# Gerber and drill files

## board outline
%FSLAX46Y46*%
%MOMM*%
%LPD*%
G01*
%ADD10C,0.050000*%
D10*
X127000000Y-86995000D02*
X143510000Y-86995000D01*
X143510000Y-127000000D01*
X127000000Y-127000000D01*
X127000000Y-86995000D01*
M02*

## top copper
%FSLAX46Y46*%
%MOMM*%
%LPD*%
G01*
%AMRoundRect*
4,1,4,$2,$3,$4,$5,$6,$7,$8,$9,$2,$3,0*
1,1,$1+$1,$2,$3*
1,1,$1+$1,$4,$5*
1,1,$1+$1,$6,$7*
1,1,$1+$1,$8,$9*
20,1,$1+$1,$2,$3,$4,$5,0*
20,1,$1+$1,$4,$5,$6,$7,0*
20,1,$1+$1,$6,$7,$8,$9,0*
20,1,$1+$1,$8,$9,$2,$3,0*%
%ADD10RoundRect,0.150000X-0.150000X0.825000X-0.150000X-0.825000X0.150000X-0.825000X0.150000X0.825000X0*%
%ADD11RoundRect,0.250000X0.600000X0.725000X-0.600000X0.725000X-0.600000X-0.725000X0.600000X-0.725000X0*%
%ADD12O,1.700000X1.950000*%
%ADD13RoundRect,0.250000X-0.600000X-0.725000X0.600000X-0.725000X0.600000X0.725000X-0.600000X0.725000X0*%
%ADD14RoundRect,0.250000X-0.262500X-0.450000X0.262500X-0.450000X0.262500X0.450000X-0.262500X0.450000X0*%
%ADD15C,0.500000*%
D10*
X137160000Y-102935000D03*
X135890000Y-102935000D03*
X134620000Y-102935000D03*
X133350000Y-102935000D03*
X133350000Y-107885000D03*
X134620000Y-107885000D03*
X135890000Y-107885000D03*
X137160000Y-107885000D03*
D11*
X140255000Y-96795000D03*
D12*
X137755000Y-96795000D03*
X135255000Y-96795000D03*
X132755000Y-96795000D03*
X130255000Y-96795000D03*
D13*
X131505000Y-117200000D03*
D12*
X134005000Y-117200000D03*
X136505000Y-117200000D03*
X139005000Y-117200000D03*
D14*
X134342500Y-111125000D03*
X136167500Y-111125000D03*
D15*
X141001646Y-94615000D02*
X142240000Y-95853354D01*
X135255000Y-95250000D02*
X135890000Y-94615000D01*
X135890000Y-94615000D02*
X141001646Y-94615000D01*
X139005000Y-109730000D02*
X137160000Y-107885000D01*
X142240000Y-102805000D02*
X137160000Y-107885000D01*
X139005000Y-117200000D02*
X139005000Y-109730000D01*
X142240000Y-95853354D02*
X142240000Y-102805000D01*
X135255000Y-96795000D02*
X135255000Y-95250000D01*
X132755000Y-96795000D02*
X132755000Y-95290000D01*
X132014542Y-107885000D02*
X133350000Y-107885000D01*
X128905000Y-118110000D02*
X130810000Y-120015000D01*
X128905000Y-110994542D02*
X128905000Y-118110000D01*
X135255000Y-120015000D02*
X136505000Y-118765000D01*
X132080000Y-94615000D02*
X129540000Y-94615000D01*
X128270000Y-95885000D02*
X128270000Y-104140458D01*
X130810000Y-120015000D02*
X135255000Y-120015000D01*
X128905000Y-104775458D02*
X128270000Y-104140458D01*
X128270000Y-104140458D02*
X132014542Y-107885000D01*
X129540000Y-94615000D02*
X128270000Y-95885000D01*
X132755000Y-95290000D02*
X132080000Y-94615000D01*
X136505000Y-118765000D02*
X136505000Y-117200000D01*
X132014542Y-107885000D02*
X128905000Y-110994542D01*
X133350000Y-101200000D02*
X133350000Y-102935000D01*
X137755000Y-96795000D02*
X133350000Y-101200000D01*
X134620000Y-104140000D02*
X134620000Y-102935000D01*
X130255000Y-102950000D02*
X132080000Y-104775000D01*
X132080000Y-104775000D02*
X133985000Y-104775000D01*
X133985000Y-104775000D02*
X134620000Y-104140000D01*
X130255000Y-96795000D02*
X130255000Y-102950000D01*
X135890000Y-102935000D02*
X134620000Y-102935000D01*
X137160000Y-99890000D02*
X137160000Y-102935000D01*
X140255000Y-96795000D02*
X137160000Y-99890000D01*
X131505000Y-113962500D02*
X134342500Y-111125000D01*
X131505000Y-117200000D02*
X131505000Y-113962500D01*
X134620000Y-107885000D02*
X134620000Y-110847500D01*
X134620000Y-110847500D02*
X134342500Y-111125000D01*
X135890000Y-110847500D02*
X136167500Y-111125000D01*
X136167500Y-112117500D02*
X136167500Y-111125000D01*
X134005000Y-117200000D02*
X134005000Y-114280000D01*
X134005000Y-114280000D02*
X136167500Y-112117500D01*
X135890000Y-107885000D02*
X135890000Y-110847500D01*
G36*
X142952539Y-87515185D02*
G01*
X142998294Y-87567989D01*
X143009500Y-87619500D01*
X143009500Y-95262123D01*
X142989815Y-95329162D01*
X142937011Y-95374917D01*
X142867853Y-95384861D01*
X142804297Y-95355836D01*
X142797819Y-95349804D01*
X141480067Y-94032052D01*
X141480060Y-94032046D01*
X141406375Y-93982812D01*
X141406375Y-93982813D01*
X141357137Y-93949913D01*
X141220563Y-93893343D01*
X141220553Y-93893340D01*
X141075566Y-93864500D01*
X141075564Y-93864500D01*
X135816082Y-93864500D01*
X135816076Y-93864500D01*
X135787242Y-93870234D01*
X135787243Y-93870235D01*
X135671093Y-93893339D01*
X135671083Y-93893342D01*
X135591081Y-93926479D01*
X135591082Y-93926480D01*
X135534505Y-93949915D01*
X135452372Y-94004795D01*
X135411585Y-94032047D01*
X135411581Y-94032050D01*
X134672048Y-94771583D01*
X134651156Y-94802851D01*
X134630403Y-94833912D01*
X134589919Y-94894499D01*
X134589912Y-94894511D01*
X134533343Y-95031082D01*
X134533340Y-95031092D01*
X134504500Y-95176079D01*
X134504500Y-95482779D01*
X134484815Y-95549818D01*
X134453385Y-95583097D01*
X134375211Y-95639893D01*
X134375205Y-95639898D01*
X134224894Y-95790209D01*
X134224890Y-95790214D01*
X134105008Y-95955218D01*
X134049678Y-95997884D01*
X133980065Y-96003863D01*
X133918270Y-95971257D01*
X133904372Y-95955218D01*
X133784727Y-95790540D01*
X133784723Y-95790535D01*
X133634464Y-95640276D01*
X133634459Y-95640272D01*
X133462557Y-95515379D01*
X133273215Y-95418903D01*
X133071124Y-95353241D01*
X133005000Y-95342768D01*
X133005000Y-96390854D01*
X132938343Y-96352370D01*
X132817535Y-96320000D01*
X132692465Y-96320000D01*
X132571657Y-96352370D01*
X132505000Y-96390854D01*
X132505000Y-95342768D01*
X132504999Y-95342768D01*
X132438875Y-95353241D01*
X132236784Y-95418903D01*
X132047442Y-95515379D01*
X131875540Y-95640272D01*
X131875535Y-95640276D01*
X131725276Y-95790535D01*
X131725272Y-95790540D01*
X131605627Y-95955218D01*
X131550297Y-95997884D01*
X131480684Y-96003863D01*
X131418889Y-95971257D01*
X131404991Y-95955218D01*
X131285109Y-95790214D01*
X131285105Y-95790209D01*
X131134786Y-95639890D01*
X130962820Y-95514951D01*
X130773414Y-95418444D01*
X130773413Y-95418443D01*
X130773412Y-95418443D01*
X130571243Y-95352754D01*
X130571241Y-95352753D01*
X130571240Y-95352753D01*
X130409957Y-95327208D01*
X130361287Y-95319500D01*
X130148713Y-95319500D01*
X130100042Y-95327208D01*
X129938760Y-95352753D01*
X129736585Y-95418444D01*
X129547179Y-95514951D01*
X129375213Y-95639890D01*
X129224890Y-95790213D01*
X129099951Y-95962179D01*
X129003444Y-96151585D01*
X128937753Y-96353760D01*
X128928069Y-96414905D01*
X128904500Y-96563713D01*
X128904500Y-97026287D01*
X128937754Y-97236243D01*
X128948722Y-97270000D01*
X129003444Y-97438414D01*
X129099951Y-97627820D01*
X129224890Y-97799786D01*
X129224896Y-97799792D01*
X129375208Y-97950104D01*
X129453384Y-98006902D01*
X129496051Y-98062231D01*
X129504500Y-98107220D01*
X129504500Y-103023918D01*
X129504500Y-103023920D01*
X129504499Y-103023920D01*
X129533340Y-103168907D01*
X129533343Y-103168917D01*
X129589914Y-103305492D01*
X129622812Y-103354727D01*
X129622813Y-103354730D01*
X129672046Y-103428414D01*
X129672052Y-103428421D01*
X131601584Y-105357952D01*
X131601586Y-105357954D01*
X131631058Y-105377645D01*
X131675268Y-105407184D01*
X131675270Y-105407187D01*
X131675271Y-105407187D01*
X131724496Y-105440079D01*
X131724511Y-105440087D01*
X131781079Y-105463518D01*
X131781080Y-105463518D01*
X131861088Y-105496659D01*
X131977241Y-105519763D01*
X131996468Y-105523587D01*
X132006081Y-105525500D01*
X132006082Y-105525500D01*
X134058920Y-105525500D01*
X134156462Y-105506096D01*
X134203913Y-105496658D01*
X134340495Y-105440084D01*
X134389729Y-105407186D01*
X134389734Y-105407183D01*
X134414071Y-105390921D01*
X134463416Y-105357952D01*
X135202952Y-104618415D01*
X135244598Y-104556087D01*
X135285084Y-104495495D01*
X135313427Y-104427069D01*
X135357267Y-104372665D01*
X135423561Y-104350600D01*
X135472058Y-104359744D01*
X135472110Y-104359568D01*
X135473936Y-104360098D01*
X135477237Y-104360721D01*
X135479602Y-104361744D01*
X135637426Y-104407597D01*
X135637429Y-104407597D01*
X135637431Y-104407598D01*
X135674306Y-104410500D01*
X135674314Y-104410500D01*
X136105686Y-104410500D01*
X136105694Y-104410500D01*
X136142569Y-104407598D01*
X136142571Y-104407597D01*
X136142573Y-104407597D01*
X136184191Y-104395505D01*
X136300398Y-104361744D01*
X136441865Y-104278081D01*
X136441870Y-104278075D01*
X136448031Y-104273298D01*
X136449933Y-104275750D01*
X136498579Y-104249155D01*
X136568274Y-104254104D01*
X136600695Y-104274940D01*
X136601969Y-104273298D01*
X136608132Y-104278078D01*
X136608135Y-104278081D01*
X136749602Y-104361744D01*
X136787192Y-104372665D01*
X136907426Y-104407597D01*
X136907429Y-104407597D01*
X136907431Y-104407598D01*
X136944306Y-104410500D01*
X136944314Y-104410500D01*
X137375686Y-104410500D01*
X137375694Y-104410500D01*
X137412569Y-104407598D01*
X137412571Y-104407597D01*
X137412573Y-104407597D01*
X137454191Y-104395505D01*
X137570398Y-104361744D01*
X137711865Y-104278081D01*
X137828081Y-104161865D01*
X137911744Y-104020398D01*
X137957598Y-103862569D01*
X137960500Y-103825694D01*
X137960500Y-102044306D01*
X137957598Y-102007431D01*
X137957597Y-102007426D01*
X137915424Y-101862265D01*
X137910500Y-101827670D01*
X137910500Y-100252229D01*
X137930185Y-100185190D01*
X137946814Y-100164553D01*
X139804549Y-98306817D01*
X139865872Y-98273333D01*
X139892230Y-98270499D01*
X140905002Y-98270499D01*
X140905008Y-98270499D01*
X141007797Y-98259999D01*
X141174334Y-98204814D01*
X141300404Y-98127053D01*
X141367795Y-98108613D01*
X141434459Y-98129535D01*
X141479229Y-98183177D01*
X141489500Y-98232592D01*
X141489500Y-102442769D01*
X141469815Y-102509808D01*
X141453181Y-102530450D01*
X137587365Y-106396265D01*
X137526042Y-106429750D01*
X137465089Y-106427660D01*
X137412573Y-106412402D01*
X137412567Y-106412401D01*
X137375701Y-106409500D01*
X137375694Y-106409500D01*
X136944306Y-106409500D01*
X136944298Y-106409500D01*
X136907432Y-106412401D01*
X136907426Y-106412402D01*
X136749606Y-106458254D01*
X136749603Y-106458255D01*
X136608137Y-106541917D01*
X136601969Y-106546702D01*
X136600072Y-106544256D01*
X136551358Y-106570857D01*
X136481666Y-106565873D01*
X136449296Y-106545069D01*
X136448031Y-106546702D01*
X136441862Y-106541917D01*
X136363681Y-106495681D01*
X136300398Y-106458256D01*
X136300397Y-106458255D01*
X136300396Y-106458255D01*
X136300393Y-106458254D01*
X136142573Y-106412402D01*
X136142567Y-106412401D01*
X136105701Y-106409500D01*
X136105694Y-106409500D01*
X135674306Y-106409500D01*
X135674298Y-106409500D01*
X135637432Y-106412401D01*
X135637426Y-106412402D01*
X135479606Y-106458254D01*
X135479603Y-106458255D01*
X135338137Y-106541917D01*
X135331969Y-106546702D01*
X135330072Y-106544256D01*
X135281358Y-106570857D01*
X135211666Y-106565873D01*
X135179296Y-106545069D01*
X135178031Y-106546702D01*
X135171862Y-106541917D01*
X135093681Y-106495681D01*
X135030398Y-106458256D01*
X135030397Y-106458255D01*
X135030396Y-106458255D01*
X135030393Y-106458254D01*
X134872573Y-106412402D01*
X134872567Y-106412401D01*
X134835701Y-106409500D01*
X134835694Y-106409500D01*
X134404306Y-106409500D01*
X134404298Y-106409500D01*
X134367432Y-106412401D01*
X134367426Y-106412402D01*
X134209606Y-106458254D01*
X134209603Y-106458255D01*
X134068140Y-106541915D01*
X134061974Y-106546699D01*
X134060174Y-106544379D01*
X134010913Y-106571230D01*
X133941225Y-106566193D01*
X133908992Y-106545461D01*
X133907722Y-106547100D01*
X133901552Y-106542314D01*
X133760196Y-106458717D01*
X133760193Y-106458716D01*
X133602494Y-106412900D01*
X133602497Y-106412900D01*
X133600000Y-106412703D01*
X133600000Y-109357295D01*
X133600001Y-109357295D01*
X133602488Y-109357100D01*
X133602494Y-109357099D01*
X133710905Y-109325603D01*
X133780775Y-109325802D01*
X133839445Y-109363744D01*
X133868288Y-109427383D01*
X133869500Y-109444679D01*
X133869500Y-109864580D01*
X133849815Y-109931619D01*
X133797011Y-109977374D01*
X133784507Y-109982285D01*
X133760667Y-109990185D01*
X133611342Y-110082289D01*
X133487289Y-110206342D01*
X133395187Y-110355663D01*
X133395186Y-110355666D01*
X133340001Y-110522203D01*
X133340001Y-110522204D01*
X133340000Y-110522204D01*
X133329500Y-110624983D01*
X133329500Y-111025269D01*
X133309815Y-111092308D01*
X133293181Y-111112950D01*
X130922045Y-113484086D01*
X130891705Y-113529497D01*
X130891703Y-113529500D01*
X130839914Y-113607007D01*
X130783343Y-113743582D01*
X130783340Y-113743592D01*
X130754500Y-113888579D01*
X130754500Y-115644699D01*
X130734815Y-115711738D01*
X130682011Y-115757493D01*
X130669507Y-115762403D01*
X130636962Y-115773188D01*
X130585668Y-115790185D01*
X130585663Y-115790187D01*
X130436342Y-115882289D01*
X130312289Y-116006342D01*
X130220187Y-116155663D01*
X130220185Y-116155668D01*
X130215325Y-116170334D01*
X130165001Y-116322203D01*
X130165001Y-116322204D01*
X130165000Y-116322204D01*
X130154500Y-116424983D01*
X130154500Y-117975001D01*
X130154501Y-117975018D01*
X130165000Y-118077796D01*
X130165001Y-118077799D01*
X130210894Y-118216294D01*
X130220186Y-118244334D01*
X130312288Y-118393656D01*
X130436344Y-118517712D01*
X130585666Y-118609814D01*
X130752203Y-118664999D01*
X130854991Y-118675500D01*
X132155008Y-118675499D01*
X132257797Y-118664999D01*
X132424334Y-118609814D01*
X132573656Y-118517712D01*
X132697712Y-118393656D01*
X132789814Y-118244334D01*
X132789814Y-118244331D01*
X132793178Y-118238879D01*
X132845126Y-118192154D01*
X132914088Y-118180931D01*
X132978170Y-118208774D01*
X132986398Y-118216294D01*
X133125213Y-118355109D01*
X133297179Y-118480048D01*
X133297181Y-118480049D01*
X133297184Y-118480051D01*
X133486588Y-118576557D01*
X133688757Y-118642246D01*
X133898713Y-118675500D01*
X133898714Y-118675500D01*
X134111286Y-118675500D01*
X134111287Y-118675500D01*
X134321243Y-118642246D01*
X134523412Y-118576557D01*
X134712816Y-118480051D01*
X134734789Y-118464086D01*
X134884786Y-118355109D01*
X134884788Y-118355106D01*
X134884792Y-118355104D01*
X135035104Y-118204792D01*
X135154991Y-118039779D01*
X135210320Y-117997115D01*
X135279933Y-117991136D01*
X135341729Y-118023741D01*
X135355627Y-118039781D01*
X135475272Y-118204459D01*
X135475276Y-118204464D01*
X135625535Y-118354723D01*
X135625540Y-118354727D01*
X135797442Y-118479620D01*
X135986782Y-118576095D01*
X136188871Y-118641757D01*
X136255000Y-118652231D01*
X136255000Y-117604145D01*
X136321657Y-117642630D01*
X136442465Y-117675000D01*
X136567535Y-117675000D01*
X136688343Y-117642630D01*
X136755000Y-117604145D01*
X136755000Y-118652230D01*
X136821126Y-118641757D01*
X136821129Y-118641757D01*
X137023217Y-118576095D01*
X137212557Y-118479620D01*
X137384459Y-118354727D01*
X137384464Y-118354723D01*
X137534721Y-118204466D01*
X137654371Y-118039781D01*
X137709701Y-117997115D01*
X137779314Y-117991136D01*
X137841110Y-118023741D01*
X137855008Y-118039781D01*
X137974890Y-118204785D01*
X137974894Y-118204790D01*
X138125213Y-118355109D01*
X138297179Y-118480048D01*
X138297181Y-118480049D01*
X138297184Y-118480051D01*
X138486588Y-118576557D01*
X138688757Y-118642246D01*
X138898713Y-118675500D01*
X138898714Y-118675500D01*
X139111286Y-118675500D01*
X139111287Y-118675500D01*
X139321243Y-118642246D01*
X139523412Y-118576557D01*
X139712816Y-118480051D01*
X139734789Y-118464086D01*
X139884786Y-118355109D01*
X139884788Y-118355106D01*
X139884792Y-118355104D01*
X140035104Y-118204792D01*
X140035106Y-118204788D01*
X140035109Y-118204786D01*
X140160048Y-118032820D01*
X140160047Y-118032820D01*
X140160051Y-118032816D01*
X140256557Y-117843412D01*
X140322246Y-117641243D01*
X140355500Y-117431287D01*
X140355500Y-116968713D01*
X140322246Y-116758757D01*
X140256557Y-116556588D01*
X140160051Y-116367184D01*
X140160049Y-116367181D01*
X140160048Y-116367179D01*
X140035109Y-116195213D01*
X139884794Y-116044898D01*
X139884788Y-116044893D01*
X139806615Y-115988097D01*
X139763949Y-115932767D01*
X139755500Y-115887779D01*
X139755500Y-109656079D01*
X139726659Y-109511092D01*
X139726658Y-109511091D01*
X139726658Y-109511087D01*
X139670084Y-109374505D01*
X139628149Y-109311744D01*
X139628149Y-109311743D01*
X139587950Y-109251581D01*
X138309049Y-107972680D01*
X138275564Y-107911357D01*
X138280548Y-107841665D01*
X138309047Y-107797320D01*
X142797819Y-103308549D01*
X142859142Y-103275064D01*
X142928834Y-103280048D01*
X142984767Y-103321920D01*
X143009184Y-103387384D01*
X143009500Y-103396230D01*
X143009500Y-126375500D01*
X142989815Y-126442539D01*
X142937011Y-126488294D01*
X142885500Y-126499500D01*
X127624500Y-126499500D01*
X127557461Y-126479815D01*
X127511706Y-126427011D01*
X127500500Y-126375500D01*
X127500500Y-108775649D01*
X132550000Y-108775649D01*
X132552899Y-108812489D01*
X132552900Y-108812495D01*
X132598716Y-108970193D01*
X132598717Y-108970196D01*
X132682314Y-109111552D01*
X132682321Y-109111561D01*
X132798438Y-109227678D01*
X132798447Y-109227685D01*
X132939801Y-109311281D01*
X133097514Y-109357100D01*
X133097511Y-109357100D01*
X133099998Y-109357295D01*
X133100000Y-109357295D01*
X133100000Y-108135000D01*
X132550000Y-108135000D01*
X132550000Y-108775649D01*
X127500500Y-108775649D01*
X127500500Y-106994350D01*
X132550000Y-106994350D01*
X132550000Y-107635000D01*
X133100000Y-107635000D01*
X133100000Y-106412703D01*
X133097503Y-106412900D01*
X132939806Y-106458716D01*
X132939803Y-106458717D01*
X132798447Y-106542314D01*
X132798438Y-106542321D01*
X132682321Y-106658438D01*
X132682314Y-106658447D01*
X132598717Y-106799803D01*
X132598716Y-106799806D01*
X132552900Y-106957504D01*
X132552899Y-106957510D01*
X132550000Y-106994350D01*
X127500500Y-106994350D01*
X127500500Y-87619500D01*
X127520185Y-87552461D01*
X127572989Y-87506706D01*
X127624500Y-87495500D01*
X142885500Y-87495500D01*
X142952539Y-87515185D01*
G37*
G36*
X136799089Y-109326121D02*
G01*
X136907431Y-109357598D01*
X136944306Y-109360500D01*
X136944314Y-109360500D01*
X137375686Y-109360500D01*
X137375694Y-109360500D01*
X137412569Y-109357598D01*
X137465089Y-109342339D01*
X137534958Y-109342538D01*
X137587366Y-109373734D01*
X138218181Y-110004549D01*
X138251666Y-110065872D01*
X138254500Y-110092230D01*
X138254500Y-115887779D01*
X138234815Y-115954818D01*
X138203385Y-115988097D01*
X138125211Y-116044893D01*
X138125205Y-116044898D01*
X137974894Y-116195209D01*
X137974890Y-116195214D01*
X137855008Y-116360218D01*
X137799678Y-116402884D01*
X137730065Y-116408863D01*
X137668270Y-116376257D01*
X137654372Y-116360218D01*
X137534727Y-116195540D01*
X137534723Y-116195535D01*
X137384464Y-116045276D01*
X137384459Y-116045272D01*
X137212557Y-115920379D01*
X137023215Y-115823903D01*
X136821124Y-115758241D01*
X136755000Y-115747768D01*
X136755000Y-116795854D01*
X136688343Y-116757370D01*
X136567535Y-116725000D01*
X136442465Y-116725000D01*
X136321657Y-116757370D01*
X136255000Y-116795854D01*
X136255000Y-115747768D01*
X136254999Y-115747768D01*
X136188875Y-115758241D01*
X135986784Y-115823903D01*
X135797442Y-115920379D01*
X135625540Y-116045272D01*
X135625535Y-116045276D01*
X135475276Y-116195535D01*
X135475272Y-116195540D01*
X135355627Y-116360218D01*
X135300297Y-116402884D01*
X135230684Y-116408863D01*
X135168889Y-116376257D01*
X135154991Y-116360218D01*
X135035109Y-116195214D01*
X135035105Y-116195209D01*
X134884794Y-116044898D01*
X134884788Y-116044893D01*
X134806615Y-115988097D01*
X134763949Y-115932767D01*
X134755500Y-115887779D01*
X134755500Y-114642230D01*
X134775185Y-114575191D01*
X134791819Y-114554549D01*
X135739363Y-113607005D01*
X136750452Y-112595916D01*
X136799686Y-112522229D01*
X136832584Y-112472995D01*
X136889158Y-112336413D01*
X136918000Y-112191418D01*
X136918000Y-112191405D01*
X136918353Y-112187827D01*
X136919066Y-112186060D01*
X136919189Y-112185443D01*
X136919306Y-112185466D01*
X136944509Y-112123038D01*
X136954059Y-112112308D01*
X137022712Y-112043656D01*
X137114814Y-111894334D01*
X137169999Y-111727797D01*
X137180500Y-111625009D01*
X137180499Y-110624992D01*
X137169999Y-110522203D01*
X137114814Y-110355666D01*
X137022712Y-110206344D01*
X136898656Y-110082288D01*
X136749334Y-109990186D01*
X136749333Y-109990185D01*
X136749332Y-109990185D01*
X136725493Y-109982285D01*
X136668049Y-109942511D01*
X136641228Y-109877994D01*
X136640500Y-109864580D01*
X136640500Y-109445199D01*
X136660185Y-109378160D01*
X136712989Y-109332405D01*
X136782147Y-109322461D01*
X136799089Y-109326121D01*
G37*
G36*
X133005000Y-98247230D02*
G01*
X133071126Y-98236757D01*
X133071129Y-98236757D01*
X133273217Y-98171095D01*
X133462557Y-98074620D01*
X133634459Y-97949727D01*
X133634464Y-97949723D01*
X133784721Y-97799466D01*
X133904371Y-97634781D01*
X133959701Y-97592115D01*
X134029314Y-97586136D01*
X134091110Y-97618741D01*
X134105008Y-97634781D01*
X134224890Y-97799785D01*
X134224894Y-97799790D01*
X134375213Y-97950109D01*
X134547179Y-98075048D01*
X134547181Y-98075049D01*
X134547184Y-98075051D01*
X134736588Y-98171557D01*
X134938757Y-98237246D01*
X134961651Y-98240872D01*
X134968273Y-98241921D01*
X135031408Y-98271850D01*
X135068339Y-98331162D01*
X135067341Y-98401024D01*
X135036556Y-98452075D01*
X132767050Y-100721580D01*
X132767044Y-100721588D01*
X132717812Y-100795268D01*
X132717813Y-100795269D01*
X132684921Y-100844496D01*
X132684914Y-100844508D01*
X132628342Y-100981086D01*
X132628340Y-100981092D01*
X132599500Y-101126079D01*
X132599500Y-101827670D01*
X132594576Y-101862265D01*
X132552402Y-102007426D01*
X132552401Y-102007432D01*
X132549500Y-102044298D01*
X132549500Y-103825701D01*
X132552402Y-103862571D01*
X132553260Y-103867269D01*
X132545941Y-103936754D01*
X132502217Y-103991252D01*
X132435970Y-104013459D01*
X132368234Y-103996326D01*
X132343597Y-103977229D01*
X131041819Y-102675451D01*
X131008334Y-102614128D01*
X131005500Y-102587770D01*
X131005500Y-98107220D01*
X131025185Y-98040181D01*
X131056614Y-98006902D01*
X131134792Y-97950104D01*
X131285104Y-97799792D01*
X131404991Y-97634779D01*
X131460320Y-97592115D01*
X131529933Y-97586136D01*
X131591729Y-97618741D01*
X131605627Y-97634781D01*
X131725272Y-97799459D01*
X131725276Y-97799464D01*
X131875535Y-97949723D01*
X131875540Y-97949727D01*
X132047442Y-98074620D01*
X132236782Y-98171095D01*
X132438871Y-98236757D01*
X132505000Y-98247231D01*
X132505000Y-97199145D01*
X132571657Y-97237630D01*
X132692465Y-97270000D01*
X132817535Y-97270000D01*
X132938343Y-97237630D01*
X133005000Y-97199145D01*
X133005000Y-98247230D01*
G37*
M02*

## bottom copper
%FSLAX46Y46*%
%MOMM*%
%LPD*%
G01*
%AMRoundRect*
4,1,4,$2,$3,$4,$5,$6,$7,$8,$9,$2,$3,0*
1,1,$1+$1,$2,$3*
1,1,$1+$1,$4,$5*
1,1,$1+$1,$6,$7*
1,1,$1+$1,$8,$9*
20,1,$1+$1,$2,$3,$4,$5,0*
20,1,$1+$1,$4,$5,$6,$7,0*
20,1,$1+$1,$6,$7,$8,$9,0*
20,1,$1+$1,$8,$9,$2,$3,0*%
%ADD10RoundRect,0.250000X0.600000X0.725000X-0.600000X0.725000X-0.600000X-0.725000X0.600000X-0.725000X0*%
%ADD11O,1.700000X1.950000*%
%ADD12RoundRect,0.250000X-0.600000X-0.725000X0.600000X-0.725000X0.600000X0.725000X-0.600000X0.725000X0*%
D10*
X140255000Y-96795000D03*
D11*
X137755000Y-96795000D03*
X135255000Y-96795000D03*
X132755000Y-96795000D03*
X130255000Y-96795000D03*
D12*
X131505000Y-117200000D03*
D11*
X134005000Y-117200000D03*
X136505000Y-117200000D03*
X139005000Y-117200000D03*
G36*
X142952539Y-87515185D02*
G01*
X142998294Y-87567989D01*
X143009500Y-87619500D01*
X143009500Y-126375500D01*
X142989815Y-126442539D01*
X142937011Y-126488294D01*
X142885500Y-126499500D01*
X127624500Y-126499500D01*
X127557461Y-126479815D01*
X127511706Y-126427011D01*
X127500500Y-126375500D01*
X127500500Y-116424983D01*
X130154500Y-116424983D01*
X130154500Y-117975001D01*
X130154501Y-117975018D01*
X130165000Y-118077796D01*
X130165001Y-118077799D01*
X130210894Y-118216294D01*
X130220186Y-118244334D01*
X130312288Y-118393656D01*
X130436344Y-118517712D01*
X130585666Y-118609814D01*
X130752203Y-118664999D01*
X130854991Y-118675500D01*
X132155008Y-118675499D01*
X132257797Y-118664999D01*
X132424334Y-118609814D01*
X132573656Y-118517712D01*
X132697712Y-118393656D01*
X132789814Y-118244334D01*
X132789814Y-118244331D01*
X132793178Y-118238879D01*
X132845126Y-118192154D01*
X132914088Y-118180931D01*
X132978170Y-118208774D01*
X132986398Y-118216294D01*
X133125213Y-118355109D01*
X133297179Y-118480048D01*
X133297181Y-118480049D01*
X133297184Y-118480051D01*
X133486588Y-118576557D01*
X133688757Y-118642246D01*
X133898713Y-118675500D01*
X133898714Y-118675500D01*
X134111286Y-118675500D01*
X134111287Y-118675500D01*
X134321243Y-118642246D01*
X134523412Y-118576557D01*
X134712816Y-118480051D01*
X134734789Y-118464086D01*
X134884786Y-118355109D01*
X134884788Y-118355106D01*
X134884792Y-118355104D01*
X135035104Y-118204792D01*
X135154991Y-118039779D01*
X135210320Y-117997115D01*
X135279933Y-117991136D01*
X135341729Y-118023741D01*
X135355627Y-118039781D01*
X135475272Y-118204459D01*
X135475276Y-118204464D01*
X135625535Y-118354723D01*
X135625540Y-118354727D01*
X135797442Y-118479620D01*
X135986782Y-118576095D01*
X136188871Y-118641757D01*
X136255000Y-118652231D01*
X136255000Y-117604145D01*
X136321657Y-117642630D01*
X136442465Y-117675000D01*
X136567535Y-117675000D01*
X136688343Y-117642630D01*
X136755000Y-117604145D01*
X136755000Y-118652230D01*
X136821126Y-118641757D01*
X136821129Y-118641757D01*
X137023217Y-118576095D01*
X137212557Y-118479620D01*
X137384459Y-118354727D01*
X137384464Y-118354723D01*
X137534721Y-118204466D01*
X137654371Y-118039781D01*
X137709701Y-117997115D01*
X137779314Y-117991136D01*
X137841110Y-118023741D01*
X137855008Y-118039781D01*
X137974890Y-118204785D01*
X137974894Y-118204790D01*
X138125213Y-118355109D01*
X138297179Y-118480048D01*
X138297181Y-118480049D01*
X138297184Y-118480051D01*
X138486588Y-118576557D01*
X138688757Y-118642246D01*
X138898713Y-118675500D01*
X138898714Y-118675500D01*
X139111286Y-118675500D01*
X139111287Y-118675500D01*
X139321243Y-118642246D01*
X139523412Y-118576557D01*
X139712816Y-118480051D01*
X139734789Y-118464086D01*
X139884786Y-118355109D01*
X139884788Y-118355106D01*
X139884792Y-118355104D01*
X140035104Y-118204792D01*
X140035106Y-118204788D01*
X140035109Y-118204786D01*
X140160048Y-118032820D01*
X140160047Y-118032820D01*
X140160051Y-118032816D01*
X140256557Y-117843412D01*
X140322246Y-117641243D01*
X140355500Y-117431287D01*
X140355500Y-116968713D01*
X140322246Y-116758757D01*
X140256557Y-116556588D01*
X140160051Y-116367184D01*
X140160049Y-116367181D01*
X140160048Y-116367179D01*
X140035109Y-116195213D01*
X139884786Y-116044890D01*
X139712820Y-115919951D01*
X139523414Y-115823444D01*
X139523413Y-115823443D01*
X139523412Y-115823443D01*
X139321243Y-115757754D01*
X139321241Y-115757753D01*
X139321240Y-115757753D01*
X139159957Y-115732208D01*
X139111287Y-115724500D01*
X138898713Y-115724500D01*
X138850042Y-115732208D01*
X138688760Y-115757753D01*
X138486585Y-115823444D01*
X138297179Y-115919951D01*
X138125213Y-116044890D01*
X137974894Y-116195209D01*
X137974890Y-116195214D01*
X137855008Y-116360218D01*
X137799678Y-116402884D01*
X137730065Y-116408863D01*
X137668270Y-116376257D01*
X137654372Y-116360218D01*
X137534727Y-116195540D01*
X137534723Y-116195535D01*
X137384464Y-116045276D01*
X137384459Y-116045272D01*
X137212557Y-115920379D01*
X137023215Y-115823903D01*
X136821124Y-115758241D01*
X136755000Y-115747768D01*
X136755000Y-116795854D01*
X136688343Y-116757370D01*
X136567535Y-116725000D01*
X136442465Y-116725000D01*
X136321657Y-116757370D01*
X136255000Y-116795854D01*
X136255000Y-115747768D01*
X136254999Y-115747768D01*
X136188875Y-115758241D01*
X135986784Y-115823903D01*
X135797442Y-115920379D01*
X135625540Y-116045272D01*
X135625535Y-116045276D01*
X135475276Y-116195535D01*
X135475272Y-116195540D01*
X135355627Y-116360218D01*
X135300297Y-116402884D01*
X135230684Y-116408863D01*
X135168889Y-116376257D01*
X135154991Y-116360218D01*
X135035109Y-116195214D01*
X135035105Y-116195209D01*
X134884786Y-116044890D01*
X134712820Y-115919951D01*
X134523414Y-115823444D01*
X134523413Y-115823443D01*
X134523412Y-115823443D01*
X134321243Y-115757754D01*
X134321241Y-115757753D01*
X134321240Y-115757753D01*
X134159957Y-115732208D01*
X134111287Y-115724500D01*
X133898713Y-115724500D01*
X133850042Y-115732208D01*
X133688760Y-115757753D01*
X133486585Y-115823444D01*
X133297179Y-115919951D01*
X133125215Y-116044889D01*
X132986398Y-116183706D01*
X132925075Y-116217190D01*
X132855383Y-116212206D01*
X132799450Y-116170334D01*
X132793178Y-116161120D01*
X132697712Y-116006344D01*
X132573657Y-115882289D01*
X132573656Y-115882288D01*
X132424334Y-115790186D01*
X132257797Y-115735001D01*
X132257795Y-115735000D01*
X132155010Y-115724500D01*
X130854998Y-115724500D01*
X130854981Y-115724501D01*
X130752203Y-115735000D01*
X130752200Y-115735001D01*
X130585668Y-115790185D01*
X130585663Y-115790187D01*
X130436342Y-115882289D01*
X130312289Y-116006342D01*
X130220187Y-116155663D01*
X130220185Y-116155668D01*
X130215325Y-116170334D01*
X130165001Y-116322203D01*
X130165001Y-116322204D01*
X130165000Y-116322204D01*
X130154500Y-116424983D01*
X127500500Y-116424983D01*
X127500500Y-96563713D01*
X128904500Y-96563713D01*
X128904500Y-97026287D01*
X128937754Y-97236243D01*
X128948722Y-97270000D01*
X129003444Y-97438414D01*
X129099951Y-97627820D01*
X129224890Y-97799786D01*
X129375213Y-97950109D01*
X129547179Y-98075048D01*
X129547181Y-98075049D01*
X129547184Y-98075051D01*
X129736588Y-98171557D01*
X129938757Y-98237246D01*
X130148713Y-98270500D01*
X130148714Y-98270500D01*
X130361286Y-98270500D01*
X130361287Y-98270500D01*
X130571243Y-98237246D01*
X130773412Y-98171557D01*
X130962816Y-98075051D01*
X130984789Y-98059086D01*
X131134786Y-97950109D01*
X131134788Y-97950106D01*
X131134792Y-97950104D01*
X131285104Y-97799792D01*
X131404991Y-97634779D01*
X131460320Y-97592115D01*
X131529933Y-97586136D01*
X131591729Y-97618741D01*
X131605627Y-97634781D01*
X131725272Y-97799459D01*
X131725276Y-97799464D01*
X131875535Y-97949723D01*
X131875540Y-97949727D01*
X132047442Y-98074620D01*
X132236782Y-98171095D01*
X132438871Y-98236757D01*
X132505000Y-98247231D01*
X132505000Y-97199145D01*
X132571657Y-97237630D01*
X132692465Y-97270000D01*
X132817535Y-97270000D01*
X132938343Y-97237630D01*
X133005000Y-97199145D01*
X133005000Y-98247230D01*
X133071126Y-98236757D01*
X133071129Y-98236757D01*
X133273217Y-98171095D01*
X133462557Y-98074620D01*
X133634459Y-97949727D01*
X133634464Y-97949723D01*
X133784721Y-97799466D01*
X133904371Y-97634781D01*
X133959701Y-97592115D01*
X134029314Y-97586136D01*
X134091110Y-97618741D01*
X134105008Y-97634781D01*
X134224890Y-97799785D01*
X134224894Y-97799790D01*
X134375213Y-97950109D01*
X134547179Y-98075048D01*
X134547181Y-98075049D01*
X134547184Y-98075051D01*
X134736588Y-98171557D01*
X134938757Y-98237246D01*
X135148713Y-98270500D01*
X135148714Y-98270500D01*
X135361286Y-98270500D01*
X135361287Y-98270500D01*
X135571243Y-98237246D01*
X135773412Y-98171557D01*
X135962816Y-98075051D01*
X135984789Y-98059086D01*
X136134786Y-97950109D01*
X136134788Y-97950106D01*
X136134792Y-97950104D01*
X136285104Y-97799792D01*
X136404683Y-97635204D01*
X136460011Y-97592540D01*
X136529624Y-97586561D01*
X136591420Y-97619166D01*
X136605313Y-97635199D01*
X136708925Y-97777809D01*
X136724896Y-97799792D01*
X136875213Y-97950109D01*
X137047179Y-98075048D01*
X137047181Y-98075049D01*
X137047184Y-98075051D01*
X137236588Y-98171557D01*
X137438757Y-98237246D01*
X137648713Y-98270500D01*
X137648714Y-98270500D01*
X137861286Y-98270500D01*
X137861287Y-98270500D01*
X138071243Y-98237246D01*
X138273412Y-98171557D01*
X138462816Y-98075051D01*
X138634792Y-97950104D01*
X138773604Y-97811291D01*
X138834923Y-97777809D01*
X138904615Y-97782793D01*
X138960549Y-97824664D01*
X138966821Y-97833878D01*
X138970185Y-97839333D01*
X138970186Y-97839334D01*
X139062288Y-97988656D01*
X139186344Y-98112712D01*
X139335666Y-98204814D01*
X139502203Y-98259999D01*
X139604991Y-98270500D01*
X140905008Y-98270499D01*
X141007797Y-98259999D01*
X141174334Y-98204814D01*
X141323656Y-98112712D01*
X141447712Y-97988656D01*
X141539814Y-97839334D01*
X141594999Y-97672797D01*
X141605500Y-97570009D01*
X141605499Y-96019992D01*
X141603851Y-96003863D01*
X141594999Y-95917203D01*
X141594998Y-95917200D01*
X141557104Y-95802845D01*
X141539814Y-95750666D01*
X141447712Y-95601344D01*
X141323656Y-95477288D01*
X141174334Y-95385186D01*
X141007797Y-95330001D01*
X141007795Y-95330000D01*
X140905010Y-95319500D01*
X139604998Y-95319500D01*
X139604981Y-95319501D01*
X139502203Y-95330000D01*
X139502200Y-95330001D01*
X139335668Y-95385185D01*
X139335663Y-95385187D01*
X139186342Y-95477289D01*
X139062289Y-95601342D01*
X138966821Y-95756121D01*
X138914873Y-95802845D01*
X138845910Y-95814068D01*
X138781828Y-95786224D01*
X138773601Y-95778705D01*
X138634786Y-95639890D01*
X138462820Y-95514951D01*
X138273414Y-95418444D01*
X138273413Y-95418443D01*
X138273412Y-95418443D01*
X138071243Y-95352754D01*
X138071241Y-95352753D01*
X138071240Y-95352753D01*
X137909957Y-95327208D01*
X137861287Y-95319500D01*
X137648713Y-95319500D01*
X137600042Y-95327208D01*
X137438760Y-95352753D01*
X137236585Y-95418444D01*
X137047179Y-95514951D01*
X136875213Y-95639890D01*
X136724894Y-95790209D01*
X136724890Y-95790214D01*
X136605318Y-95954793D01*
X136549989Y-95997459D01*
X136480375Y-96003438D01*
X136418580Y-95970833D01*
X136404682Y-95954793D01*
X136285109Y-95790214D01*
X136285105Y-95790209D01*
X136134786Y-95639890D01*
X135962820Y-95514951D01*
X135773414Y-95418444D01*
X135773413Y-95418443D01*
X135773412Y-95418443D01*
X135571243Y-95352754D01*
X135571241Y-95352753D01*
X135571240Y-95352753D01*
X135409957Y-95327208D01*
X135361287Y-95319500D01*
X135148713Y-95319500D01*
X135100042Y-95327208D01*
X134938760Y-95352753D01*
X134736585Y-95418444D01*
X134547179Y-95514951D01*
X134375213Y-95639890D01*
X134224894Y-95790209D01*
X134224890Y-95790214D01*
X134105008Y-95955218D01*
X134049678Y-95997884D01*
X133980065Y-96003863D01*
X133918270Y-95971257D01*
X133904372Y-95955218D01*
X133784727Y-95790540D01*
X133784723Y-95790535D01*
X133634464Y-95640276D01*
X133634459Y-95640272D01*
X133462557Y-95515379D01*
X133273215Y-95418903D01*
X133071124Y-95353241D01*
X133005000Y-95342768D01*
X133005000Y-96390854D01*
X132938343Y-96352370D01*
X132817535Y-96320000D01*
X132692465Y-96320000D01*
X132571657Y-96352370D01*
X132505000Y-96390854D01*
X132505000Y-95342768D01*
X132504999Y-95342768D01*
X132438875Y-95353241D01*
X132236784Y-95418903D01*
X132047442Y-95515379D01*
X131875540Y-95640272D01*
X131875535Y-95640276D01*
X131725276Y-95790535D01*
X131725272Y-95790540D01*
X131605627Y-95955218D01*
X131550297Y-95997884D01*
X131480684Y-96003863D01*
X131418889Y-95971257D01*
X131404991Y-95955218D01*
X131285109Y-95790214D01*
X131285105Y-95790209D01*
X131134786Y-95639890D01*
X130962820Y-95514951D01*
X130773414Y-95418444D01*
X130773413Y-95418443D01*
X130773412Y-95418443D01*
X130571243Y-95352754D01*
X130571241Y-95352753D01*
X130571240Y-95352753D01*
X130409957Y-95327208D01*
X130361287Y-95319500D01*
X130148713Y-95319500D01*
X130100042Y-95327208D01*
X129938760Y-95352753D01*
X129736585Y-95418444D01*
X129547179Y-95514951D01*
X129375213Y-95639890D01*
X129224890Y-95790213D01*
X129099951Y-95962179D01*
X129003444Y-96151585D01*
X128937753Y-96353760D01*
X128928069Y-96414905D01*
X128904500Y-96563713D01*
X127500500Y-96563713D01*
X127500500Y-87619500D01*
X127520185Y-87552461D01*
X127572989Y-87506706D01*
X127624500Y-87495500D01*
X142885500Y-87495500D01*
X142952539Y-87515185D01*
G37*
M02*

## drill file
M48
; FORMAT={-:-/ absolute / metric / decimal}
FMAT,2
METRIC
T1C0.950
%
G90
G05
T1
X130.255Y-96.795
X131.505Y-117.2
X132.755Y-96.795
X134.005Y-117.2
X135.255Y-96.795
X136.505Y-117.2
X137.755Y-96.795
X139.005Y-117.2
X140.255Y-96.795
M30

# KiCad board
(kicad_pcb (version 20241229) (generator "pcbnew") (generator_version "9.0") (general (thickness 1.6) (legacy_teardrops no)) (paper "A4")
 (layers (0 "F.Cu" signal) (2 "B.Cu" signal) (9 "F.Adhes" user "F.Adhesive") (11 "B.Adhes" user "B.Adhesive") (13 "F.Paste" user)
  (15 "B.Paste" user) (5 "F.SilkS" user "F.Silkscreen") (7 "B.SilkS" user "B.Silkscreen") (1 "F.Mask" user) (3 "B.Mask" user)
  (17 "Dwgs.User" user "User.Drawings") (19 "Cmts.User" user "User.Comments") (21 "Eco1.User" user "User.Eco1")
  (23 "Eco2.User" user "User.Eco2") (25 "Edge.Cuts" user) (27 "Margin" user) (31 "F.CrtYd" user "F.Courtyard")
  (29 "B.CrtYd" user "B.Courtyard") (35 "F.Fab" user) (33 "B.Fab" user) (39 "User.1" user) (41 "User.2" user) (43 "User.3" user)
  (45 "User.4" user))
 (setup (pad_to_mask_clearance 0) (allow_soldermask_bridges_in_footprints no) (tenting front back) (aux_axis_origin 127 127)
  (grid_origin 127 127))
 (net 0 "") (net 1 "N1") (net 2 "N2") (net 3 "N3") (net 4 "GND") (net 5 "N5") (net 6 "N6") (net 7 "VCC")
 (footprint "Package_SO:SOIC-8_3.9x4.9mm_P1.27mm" (layer "F.Cu") (at 135.255 105.41 -90)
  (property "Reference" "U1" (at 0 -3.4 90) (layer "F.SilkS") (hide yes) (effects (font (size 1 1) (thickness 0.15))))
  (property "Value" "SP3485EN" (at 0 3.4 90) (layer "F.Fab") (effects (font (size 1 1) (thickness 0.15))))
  (pad "1" smd roundrect (at -2.475 -1.905 270) (size 1.95 0.6) (layers "F.Cu" "F.Mask" "F.Paste") (roundrect_rratio 0.25) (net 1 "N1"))
  (pad "2" smd roundrect (at -2.475 -0.635 270) (size 1.95 0.6) (layers "F.Cu" "F.Mask" "F.Paste") (roundrect_rratio 0.25) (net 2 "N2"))
  (pad "3" smd roundrect (at -2.475 0.635 270) (size 1.95 0.6) (layers "F.Cu" "F.Mask" "F.Paste") (roundrect_rratio 0.25) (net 2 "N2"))
  (pad "4" smd roundrect (at -2.475 1.905 270) (size 1.95 0.6) (layers "F.Cu" "F.Mask" "F.Paste") (roundrect_rratio 0.25) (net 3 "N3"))
  (pad "5" smd roundrect (at 2.475 1.905 270) (size 1.95 0.6) (layers "F.Cu" "F.Mask" "F.Paste") (roundrect_rratio 0.25) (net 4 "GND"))
  (pad "6" smd roundrect (at 2.475 0.635 270) (size 1.95 0.6) (layers "F.Cu" "F.Mask" "F.Paste") (roundrect_rratio 0.25) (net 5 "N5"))
  (pad "7" smd roundrect (at 2.475 -0.635 270) (size 1.95 0.6) (layers "F.Cu" "F.Mask" "F.Paste") (roundrect_rratio 0.25) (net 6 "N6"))
  (pad "8" smd roundrect (at 2.475 -1.905 270) (size 1.95 0.6) (layers "F.Cu" "F.Mask" "F.Paste") (roundrect_rratio 0.25) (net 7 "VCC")))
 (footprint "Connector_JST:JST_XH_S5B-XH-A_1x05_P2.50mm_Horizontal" (layer "F.Cu") (at 140.255 96.795 180)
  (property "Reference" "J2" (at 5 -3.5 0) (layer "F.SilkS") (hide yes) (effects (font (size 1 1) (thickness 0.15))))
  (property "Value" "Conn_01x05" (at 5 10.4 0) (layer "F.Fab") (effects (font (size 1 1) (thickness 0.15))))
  (pad "1" thru_hole roundrect (at 0 0 180) (size 1.7 1.95) (drill 0.95) (layers "*.Cu" "*.Mask") (remove_unused_layers no)
   (roundrect_rratio 0.147059) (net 1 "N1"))
  (pad "2" thru_hole oval (at 2.5 0 180) (size 1.7 1.95) (drill 0.95) (layers "*.Cu" "*.Mask") (remove_unused_layers no) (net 3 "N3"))
  (pad "3" thru_hole oval (at 5 0 180) (size 1.7 1.95) (drill 0.95) (layers "*.Cu" "*.Mask") (remove_unused_layers no) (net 7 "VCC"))
  (pad "4" thru_hole oval (at 7.5 0 180) (size 1.7 1.95) (drill 0.95) (layers "*.Cu" "*.Mask") (remove_unused_layers no) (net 4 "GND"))
  (pad "5" thru_hole oval (at 10 0 180) (size 1.7 1.95) (drill 0.95) (layers "*.Cu" "*.Mask") (remove_unused_layers no) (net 2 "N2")))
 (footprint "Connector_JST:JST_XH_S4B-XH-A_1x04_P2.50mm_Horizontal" (layer "F.Cu") (at 131.505 117.2)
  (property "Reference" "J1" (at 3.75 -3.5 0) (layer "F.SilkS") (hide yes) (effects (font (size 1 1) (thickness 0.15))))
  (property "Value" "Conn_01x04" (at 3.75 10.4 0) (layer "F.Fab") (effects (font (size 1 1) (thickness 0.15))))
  (pad "1" thru_hole roundrect (at 0 0) (size 1.7 1.95) (drill 0.95) (layers "*.Cu" "*.Mask") (remove_unused_layers no)
   (roundrect_rratio 0.147059) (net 5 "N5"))
  (pad "2" thru_hole oval (at 2.5 0) (size 1.7 1.95) (drill 0.95) (layers "*.Cu" "*.Mask") (remove_unused_layers no) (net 6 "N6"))
  (pad "3" thru_hole oval (at 5 0) (size 1.7 1.95) (drill 0.95) (layers "*.Cu" "*.Mask") (remove_unused_layers no) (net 4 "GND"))
  (pad "4" thru_hole oval (at 7.5 0) (size 1.7 1.95) (drill 0.95) (layers "*.Cu" "*.Mask") (remove_unused_layers no) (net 7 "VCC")))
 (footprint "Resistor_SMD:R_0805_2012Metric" (layer "F.Cu") (at 135.255 111.125)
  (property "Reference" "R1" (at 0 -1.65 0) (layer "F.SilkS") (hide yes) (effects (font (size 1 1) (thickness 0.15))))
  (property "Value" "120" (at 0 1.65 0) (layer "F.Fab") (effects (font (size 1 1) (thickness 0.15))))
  (pad "1" smd roundrect (at -0.9125 0) (size 1.025 1.4) (layers "F.Cu" "F.Mask" "F.Paste") (roundrect_rratio 0.243902) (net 5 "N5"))
  (pad "2" smd roundrect (at 0.9125 0) (size 1.025 1.4) (layers "F.Cu" "F.Mask" "F.Paste") (roundrect_rratio 0.243902) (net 6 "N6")))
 (gr_rect (start 127 86.995) (end 143.51 127) (stroke (width 0.05) (type default)) (fill no) (layer "Edge.Cuts"))
 (segment (start 141.001646 94.615) (end 142.24 95.853354) (width 0.5) (layer "F.Cu") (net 7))
 (segment (start 135.255 95.25) (end 135.89 94.615) (width 0.5) (layer "F.Cu") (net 7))
 (segment (start 135.89 94.615) (end 141.001646 94.615) (width 0.5) (layer "F.Cu") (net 7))
 (segment (start 139.005 109.73) (end 137.16 107.885) (width 0.5) (layer "F.Cu") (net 7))
 (segment (start 142.24 102.805) (end 137.16 107.885) (width 0.5) (layer "F.Cu") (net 7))
 (segment (start 139.005 117.2) (end 139.005 109.73) (width 0.5) (layer "F.Cu") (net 7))
 (segment (start 142.24 95.853354) (end 142.24 102.805) (width 0.5) (layer "F.Cu") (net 7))
 (segment (start 135.255 96.795) (end 135.255 95.25) (width 0.5) (layer "F.Cu") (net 7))
 (segment (start 132.755 96.795) (end 132.755 95.29) (width 0.5) (layer "F.Cu") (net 4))
 (segment (start 132.014542 107.885) (end 133.35 107.885) (width 0.5) (layer "F.Cu") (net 4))
 (segment (start 128.905 118.11) (end 130.81 120.015) (width 0.5) (layer "F.Cu") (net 4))
 (segment (start 128.905 110.994542) (end 128.905 118.11) (width 0.5) (layer "F.Cu") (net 4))
 (segment (start 135.255 120.015) (end 136.505 118.765) (width 0.5) (layer "F.Cu") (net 4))
 (segment (start 132.08 94.615) (end 129.54 94.615) (width 0.5) (layer "F.Cu") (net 4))
 (segment (start 128.27 95.885) (end 128.27 104.140458) (width 0.5) (layer "F.Cu") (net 4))
 (segment (start 130.81 120.015) (end 135.255 120.015) (width 0.5) (layer "F.Cu") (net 4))
 (segment (start 128.905 104.775458) (end 128.27 104.140458) (width 0.5) (layer "F.Cu") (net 4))
 (segment (start 128.27 104.140458) (end 132.014542 107.885) (width 0.5) (layer "F.Cu") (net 4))
 (segment (start 129.54 94.615) (end 128.27 95.885) (width 0.5) (layer "F.Cu") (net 4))
 (segment (start 132.755 95.29) (end 132.08 94.615) (width 0.5) (layer "F.Cu") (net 4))
 (segment (start 136.505 118.765) (end 136.505 117.2) (width 0.5) (layer "F.Cu") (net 4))
 (segment (start 132.014542 107.885) (end 128.905 110.994542) (width 0.5) (layer "F.Cu") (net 4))
 (segment (start 133.35 101.2) (end 133.35 102.935) (width 0.5) (layer "F.Cu") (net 3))
 (segment (start 137.755 96.795) (end 133.35 101.2) (width 0.5) (layer "F.Cu") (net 3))
 (segment (start 134.62 104.14) (end 134.62 102.935) (width 0.5) (layer "F.Cu") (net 2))
 (segment (start 130.255 102.95) (end 132.08 104.775) (width 0.5) (layer "F.Cu") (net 2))
 (segment (start 132.08 104.775) (end 133.985 104.775) (width 0.5) (layer "F.Cu") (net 2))
 (segment (start 133.985 104.775) (end 134.62 104.14) (width 0.5) (layer "F.Cu") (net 2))
 (segment (start 130.255 96.795) (end 130.255 102.95) (width 0.5) (layer "F.Cu") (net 2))
 (segment (start 135.89 102.935) (end 134.62 102.935) (width 0.5) (layer "F.Cu") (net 2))
 (segment (start 137.16 99.89) (end 137.16 102.935) (width 0.5) (layer "F.Cu") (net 1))
 (segment (start 140.255 96.795) (end 137.16 99.89) (width 0.5) (layer "F.Cu") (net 1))
 (segment (start 131.505 113.9625) (end 134.3425 111.125) (width 0.5) (layer "F.Cu") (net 5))
 (segment (start 131.505 117.2) (end 131.505 113.9625) (width 0.5) (layer "F.Cu") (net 5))
 (segment (start 134.62 107.885) (end 134.62 110.8475) (width 0.5) (layer "F.Cu") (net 5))
 (segment (start 134.62 110.8475) (end 134.3425 111.125) (width 0.5) (layer "F.Cu") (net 5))
 (segment (start 135.89 110.8475) (end 136.1675 111.125) (width 0.5) (layer "F.Cu") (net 6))
 (segment (start 136.1675 112.1175) (end 136.1675 111.125) (width 0.5) (layer "F.Cu") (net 6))
 (segment (start 134.005 117.2) (end 134.005 114.28) (width 0.5) (layer "F.Cu") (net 6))
 (segment (start 134.005 114.28) (end 136.1675 112.1175) (width 0.5) (layer "F.Cu") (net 6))
 (segment (start 135.89 107.885) (end 135.89 110.8475) (width 0.5) (layer "F.Cu") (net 6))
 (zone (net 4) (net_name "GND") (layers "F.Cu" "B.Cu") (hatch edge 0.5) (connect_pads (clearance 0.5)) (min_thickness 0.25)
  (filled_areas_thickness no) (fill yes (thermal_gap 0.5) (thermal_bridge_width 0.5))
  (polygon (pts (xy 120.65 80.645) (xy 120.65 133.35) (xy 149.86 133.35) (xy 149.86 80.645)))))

